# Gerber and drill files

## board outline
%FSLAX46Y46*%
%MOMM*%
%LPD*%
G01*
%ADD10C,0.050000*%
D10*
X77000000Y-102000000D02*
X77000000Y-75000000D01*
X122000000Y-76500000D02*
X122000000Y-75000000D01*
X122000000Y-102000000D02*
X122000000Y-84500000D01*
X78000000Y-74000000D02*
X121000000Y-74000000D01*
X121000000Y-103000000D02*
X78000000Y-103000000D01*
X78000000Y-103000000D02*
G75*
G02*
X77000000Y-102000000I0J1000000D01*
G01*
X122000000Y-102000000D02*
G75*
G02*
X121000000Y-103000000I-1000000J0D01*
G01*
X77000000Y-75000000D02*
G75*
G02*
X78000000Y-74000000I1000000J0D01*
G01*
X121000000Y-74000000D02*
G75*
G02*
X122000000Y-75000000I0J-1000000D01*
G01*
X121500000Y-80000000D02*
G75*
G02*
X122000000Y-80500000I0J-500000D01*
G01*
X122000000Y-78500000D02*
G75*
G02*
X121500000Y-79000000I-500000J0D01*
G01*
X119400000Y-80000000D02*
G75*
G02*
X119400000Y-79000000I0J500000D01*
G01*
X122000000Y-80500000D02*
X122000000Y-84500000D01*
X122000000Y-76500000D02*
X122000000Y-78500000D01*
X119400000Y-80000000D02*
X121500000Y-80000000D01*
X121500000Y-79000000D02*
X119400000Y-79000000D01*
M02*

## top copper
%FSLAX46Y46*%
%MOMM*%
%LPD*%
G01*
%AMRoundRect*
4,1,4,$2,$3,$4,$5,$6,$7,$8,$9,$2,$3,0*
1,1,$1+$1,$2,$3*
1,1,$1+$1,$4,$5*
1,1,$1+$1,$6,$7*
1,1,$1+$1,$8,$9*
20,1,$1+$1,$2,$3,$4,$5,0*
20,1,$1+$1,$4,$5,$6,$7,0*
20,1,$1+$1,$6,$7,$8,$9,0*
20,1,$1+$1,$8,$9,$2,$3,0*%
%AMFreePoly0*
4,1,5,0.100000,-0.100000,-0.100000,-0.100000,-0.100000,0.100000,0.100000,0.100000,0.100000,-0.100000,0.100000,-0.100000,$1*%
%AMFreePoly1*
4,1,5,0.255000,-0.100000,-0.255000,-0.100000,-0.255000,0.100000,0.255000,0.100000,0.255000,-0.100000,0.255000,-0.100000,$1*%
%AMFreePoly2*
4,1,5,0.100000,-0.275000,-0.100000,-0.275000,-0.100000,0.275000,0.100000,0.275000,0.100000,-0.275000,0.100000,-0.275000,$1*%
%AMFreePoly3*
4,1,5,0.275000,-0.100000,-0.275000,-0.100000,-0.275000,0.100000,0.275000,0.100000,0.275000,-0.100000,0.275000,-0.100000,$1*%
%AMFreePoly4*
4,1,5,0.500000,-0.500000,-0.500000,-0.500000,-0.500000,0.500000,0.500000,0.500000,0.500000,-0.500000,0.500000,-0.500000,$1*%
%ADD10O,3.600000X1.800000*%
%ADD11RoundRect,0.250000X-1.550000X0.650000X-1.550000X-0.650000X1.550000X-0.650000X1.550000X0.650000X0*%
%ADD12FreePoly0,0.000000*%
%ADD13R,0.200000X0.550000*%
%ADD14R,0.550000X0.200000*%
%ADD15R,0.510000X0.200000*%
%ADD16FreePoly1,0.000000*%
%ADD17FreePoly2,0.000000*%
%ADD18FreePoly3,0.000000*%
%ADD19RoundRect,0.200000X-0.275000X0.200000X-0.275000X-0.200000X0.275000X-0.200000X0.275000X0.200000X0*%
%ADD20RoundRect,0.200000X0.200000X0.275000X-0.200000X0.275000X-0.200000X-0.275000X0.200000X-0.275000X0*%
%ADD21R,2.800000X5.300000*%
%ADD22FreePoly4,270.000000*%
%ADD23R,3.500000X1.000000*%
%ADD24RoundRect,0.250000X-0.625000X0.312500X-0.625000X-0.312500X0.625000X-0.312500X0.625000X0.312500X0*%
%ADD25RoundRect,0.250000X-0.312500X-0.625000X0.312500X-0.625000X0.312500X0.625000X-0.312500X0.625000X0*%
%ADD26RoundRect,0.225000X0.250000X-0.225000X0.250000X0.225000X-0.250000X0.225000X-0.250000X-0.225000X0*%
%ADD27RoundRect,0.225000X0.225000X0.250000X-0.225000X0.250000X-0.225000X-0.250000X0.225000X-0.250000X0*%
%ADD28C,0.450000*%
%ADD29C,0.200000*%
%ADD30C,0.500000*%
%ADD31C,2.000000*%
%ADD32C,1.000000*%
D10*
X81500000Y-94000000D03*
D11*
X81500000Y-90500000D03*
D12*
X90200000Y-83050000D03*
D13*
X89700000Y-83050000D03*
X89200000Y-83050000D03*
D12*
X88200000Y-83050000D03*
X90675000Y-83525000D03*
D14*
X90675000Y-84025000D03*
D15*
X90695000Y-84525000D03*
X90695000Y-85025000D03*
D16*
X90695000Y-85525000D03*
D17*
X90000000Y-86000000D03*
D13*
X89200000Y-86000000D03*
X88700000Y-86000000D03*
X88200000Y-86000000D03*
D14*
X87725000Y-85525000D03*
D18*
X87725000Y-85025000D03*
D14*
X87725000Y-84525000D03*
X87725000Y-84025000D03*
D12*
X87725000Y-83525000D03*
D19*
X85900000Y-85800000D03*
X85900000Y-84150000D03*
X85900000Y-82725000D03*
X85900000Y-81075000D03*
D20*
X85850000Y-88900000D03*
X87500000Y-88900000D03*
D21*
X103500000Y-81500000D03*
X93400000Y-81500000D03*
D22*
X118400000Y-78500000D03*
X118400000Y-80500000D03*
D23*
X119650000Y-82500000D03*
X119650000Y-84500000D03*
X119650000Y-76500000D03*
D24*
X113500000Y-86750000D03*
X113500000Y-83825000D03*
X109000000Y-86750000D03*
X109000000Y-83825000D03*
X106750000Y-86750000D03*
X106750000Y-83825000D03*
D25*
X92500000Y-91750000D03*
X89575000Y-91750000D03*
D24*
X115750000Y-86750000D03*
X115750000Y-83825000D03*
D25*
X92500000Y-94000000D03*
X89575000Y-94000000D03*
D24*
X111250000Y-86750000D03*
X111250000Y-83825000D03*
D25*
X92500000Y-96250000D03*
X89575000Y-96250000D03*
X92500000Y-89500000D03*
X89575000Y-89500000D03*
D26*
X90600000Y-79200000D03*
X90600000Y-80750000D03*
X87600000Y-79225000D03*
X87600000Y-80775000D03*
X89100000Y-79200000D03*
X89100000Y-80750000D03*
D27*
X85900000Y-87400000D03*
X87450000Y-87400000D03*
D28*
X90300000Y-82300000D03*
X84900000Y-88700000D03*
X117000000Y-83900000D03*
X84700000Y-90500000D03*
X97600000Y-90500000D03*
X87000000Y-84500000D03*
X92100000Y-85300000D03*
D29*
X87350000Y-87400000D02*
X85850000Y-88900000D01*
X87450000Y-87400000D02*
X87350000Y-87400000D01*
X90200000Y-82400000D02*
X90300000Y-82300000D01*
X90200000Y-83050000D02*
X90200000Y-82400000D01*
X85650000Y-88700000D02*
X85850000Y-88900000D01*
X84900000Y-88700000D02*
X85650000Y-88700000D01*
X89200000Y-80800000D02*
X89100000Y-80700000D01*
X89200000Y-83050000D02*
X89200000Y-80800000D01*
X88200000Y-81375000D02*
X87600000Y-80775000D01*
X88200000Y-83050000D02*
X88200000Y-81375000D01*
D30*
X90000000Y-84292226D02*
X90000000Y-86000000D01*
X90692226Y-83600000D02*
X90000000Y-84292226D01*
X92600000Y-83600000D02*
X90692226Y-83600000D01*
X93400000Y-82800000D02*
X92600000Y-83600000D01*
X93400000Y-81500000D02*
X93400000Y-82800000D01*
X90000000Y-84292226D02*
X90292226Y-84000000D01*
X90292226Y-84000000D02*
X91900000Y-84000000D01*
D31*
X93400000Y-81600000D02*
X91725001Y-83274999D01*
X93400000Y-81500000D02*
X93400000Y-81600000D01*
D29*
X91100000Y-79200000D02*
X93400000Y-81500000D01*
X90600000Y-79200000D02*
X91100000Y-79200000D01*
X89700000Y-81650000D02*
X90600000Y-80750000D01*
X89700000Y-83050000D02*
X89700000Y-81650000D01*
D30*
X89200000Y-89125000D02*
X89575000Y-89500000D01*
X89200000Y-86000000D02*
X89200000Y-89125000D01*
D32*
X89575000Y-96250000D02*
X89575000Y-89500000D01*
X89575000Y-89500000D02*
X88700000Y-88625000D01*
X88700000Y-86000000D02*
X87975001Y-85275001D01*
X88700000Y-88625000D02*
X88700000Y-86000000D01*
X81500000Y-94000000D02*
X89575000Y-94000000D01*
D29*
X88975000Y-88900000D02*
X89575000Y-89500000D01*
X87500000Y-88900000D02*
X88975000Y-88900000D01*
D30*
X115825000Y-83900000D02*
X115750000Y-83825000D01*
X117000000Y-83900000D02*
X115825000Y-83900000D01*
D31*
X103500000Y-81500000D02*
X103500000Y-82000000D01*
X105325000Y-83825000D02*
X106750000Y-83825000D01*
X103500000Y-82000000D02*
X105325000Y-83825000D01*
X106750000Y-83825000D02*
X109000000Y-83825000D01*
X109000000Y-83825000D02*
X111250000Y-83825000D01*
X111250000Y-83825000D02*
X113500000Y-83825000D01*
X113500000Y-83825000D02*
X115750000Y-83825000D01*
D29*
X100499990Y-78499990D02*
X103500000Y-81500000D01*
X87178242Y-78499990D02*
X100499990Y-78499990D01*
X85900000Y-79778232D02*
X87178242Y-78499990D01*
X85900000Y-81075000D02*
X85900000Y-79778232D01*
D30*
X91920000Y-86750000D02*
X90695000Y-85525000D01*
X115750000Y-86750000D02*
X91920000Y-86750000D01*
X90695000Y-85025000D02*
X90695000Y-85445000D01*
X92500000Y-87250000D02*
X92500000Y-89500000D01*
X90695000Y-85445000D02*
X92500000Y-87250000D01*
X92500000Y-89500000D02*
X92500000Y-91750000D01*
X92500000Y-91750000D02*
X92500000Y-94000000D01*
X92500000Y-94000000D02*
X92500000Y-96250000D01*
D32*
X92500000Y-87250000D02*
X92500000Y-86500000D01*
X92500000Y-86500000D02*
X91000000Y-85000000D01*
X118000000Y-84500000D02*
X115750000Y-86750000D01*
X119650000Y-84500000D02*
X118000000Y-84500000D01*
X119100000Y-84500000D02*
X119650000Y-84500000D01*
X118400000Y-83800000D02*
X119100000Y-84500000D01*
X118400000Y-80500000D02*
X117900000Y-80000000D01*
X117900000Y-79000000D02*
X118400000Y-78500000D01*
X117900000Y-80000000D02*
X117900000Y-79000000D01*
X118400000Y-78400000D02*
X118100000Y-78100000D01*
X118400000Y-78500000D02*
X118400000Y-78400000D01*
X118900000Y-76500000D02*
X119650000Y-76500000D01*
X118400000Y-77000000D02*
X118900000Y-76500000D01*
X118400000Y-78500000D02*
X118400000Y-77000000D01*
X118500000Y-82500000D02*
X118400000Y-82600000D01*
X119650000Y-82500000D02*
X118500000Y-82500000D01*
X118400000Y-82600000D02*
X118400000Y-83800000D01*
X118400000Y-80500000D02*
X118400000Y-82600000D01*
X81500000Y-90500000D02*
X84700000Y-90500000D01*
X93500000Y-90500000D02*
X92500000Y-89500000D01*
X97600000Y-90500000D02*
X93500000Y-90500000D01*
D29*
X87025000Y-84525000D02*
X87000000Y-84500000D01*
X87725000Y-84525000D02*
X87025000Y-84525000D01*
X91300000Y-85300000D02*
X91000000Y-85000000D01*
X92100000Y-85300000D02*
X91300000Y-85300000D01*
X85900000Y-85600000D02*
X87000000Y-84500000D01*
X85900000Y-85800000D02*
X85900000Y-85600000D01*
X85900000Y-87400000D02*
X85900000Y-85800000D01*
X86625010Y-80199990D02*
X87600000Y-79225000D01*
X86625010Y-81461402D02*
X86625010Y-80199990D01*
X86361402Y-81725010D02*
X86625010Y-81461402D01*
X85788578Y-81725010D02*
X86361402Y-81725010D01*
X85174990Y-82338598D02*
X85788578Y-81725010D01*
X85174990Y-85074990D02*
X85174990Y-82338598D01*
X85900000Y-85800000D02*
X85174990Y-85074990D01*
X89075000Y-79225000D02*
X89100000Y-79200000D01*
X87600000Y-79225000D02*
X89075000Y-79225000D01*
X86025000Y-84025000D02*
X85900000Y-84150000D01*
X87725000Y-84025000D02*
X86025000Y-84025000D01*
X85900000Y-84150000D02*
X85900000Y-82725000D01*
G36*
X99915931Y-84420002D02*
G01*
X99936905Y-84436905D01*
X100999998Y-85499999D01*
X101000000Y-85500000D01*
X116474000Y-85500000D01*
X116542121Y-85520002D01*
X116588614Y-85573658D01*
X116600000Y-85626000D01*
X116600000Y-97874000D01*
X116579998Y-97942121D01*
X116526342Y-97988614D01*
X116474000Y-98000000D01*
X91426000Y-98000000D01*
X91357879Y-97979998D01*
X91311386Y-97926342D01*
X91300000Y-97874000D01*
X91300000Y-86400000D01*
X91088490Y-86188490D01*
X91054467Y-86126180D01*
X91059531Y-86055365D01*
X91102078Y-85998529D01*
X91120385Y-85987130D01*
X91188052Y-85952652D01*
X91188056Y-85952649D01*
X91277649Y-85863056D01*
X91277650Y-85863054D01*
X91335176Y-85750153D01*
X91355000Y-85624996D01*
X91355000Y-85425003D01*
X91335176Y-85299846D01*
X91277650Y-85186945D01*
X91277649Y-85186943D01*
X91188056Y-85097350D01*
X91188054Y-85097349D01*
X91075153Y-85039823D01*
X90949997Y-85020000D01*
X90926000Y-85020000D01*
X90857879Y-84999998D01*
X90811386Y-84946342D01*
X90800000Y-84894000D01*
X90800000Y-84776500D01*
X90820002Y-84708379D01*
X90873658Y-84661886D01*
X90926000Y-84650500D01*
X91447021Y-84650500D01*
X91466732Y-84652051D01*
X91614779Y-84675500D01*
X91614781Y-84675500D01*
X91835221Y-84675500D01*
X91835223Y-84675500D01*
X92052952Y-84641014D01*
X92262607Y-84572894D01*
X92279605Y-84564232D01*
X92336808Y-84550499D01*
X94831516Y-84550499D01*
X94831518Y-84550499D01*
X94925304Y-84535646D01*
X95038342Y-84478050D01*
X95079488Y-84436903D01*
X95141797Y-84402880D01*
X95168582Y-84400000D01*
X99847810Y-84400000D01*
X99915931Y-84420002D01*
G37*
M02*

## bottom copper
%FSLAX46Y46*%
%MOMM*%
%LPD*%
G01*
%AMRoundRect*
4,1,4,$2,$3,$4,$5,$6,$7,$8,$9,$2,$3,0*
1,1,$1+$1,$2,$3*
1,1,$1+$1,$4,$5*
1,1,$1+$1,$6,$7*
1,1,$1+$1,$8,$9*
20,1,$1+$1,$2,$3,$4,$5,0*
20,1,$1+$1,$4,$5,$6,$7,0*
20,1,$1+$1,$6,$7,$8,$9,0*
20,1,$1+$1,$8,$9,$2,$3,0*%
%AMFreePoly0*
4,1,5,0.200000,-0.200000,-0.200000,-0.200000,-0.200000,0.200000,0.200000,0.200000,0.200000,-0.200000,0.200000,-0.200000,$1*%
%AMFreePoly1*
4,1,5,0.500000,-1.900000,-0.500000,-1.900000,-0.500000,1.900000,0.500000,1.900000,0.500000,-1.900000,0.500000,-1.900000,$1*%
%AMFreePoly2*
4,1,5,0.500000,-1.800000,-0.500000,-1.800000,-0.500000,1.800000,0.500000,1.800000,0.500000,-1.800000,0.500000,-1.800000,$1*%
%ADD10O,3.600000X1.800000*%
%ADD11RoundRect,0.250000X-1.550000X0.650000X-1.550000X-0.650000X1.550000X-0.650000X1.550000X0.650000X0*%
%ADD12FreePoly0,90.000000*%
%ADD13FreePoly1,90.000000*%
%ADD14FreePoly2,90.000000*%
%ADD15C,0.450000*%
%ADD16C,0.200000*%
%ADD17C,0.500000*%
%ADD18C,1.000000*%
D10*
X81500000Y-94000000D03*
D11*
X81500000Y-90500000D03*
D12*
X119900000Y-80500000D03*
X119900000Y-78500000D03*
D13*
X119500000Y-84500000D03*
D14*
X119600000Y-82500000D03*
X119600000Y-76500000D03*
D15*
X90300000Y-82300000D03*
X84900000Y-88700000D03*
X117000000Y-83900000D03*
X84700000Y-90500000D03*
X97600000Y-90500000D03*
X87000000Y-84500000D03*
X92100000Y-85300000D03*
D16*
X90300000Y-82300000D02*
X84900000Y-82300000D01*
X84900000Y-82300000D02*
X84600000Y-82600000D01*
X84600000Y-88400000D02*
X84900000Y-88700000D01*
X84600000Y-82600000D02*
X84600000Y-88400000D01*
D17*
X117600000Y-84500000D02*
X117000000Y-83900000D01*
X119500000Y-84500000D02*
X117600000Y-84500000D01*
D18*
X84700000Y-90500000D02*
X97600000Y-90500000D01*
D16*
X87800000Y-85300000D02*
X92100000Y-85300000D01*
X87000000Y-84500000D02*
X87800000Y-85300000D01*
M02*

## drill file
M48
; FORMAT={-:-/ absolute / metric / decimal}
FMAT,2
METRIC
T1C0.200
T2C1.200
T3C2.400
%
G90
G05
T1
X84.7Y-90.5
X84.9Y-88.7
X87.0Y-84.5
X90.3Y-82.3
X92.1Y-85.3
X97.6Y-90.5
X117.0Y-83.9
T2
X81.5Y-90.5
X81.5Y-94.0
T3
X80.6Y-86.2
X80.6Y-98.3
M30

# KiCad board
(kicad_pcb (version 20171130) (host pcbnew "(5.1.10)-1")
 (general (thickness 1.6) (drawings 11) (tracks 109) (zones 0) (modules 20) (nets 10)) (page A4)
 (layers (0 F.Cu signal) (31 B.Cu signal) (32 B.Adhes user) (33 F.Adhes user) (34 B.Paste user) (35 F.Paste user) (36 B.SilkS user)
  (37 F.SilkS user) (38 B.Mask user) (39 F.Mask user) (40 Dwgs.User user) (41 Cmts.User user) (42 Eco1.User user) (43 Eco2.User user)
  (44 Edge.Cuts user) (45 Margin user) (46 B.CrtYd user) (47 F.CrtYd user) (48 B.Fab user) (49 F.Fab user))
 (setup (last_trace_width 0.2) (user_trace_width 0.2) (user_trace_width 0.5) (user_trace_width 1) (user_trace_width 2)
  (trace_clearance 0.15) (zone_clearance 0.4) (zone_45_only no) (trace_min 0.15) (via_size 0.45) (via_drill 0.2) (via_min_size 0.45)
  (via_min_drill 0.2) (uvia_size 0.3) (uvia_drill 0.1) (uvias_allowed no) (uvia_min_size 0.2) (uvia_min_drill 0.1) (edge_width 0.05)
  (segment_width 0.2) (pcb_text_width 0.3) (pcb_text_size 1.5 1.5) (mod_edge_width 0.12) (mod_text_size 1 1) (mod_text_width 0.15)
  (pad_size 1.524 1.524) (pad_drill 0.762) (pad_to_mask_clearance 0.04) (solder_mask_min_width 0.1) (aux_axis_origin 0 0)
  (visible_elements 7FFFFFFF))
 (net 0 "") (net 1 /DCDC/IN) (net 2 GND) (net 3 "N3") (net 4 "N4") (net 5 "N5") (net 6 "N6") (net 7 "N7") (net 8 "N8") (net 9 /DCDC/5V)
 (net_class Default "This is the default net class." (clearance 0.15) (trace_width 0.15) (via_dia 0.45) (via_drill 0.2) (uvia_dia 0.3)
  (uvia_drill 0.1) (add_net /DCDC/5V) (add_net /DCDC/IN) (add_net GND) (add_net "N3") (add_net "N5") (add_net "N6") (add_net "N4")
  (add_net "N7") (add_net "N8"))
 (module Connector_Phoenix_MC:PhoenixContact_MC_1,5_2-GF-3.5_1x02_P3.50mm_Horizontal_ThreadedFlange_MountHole (layer F.Cu)
  (at 81.5 90.5 270)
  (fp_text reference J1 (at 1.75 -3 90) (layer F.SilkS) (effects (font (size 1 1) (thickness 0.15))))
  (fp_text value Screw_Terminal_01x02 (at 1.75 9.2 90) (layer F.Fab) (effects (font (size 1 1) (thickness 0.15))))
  (pad "" np_thru_hole circle (at 7.8 0.9 270) (size 2.4 2.4) (drill 2.4) (layers *.Cu *.Mask))
  (pad "" np_thru_hole circle (at -4.3 0.9 270) (size 2.4 2.4) (drill 2.4) (layers *.Cu *.Mask))
  (pad 2 thru_hole oval (at 3.5 0 270) (size 1.8 3.6) (drill 1.2) (layers *.Cu *.Mask) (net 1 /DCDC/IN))
  (pad 1 thru_hole roundrect (at 0 0 270) (size 1.8 3.6) (drill 1.2) (layers *.Cu *.Mask) (roundrect_rratio 0.138889) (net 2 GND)))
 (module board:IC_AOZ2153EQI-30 (layer F.Cu) (at 89.2 84.525)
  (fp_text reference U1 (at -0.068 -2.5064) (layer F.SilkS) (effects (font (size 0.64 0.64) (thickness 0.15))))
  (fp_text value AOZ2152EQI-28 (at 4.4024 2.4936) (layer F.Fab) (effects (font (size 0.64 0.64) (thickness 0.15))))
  (pad 15 smd custom (at 1 -1.475) (size 0.2 0.2) (layers F.Cu) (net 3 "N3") (zone_connect 0) (options (clearance outline) (anchor rect))
   (primitives))
  (pad 16 smd rect (at 0.5 -1.475) (size 0.2 0.55) (layers F.Cu F.Paste F.Mask) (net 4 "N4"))
  (pad 17 smd rect (at 0 -1.475) (size 0.2 0.55) (layers F.Cu F.Paste F.Mask) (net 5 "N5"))
  (pad 18 smd custom (at -1 -1.475) (size 0.2 0.2) (layers F.Cu) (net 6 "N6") (zone_connect 0) (options (clearance outline) (anchor rect))
   (primitives))
  (pad 14 smd custom (at 1.475 -1) (size 0.2 0.2) (layers F.Cu) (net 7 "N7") (zone_connect 0) (options (clearance outline) (anchor rect))
   (primitives))
  (pad 13 smd rect (at 1.475 -0.5) (size 0.55 0.2) (layers F.Cu F.Paste) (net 7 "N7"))
  (pad 12 smd rect (at 1.495 0) (size 0.51 0.2) (layers F.Cu F.Paste) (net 2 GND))
  (pad 11 smd rect (at 1.495 0.5) (size 0.51 0.2) (layers F.Cu F.Paste) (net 2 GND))
  (pad 10 smd custom (at 1.495 1) (size 0.51 0.2) (layers F.Cu F.Paste) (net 2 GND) (zone_connect 0)
   (options (clearance outline) (anchor rect)) (primitives))
  (pad 9 smd custom (at 0.8 1.475) (size 0.2 0.55) (layers F.Cu F.Paste) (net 7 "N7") (zone_connect 0)
   (options (clearance outline) (anchor rect)) (primitives))
  (pad 8 smd rect (at 0 1.475) (size 0.2 0.55) (layers F.Cu F.Paste) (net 1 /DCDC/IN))
  (pad 7 smd rect (at -0.5 1.475) (size 0.2 0.55) (layers F.Cu F.Paste) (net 1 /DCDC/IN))
  (pad 6 smd rect (at -1 1.475) (size 0.2 0.55) (layers F.Cu F.Paste) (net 1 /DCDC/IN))
  (pad 5 smd rect (at -1.475 1) (size 0.55 0.2) (layers F.Cu F.Paste) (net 1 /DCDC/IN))
  (pad 4 smd custom (at -1.475 0.5) (size 0.55 0.2) (layers F.Cu F.Paste) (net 1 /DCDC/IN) (zone_connect 0)
   (options (clearance outline) (anchor rect)) (primitives))
  (pad 3 smd rect (at -1.475 0) (size 0.55 0.2) (layers F.Cu F.Paste F.Mask) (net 2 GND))
  (pad 2 smd rect (at -1.475 -0.5) (size 0.55 0.2) (layers F.Cu F.Paste F.Mask) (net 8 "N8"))
  (pad 1 smd custom (at -1.475 -1) (size 0.2 0.2) (layers F.Cu) (zone_connect 0) (options (clearance outline) (anchor rect)) (primitives)))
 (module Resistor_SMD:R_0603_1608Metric (layer F.Cu) (at 85.9 84.975 270)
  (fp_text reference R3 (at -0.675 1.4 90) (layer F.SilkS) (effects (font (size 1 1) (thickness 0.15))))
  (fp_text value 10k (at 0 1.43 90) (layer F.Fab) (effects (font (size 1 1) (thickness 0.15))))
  (pad 2 smd roundrect (at 0.825 0 270) (size 0.8 0.95) (layers F.Cu F.Paste F.Mask) (roundrect_rratio 0.25) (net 2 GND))
  (pad 1 smd roundrect (at -0.825 0 270) (size 0.8 0.95) (layers F.Cu F.Paste F.Mask) (roundrect_rratio 0.25) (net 8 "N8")))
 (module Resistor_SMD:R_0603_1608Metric (layer F.Cu) (at 85.9 81.9 270)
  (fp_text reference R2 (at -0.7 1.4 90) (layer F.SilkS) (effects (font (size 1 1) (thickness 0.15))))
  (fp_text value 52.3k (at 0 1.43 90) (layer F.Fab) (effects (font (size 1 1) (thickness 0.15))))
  (pad 2 smd roundrect (at 0.825 0 270) (size 0.8 0.95) (layers F.Cu F.Paste F.Mask) (roundrect_rratio 0.25) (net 8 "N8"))
  (pad 1 smd roundrect (at -0.825 0 270) (size 0.8 0.95) (layers F.Cu F.Paste F.Mask) (roundrect_rratio 0.25) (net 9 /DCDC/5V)))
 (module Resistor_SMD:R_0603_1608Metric (layer F.Cu) (at 86.675 88.9 180)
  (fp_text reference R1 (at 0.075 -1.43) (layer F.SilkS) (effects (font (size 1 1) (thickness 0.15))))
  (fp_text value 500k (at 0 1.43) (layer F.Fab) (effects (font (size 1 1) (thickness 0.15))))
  (pad 2 smd roundrect (at 0.825 0 180) (size 0.8 0.95) (layers F.Cu F.Paste F.Mask) (roundrect_rratio 0.25) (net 3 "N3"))
  (pad 1 smd roundrect (at -0.825 0 180) (size 0.8 0.95) (layers F.Cu F.Paste F.Mask) (roundrect_rratio 0.25) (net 1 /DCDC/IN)))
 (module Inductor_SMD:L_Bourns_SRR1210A (layer F.Cu) (at 98.45 81.5 180)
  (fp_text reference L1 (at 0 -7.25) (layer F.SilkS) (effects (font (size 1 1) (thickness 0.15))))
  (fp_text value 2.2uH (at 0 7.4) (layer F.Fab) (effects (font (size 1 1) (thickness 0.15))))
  (pad 1 smd rect (at -5.05 0 180) (size 2.8 5.3) (layers F.Cu F.Paste F.Mask) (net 9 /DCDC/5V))
  (pad 2 smd rect (at 5.05 0 180) (size 2.8 5.3) (layers F.Cu F.Paste F.Mask) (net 7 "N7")))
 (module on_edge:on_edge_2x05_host (layer F.Cu) (at 122 80.5 270)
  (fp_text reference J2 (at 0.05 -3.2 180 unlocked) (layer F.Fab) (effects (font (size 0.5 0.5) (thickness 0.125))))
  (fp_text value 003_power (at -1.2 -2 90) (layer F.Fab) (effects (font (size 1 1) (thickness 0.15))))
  (fp_arc (start 0 0.5) (end 0 0) (angle -90) (layer Edge.Cuts) (width 0.05))
  (fp_arc (start -2 0.5) (end -1.5 0.5) (angle -90) (layer Edge.Cuts) (width 0.05))
  (fp_arc (start -1 2.6) (end -1.5 2.6) (angle -180) (layer Edge.Cuts) (width 0.05))
  (fp_line (start 0 0) (end 4 0) (layer Edge.Cuts) (width 0.05))
  (fp_line (start -4 0) (end -2 0) (layer Edge.Cuts) (width 0.05))
  (fp_line (start -0.5 2.6) (end -0.5 0.5) (layer Edge.Cuts) (width 0.05))
  (fp_line (start -1.5 0.5) (end -1.5 2.6) (layer Edge.Cuts) (width 0.05))
  (pad 2 smd custom (at -2 3.6 270) (size 1 1) (layers F.Cu F.Mask) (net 2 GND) (zone_connect 0) (options (clearance outline) (anchor rect))
   (primitives))
  (pad 3 smd custom (at 0 3.6 270) (size 1 1) (layers F.Cu F.Mask) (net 2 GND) (zone_connect 0) (options (clearance outline) (anchor rect))
   (primitives))
  (pad 8 smd custom (at 0 2.1 90) (size 0.4 0.4) (layers B.Cu B.Mask) (zone_connect 0) (options (clearance outline) (anchor rect))
   (primitives))
  (pad 7 smd custom (at -2 2.1 90) (size 0.4 0.4) (layers B.Cu B.Mask) (zone_connect 0) (options (clearance outline) (anchor rect))
   (primitives))
  (pad 4 smd rect (at 2 2.35 270) (size 1 3.5) (layers F.Cu F.Mask) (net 2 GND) (zone_connect 0))
  (pad 10 smd custom (at 4 2.5 90) (size 1 3.8) (layers B.Cu B.Mask) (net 9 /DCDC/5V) (zone_connect 0)
   (options (clearance outline) (anchor rect)) (primitives))
  (pad 9 smd custom (at 2 2.4 90) (size 1 3.6) (layers B.Cu B.Mask) (zone_connect 0) (options (clearance outline) (anchor rect))
   (primitives))
  (pad 6 smd custom (at -4 2.4 90) (size 1 3.6) (layers B.Cu B.Mask) (zone_connect 0) (options (clearance outline) (anchor rect))
   (primitives))
  (pad 5 smd rect (at 4 2.35 270) (size 1 3.5) (layers F.Cu F.Mask) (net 2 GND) (zone_connect 0))
  (pad 1 smd rect (at -4 2.35 270) (size 1 3.5) (layers F.Cu F.Mask) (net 2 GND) (zone_connect 0)))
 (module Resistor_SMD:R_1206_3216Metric (layer F.Cu) (at 113.5 85.2875 270)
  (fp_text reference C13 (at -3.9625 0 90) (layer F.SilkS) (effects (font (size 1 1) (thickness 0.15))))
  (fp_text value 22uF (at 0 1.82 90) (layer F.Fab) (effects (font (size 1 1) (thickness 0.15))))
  (pad 2 smd roundrect (at 1.4625 0 270) (size 1.125 1.75) (layers F.Cu F.Paste F.Mask) (roundrect_rratio 0.222222) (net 2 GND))
  (pad 1 smd roundrect (at -1.4625 0 270) (size 1.125 1.75) (layers F.Cu F.Paste F.Mask) (roundrect_rratio 0.222222) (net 9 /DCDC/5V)))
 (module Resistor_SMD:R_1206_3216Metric (layer F.Cu) (at 109 85.2875 270)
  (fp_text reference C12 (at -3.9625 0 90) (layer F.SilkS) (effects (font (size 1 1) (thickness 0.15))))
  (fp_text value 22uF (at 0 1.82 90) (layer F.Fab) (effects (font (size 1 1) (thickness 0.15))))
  (pad 2 smd roundrect (at 1.4625 0 270) (size 1.125 1.75) (layers F.Cu F.Paste F.Mask) (roundrect_rratio 0.222222) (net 2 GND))
  (pad 1 smd roundrect (at -1.4625 0 270) (size 1.125 1.75) (layers F.Cu F.Paste F.Mask) (roundrect_rratio 0.222222) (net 9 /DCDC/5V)))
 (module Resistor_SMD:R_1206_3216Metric (layer F.Cu) (at 106.75 85.2875 270)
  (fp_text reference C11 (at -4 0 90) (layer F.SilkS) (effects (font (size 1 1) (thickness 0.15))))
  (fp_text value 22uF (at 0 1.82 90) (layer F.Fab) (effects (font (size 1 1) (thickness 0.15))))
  (pad 2 smd roundrect (at 1.4625 0 270) (size 1.125 1.75) (layers F.Cu F.Paste F.Mask) (roundrect_rratio 0.222222) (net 2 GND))
  (pad 1 smd roundrect (at -1.4625 0 270) (size 1.125 1.75) (layers F.Cu F.Paste F.Mask) (roundrect_rratio 0.222222) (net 9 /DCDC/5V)))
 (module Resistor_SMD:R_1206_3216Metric (layer F.Cu) (at 91.0375 91.75)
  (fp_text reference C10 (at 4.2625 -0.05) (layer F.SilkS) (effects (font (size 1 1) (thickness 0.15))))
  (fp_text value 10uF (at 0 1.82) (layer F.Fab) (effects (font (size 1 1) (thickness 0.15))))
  (pad 2 smd roundrect (at 1.4625 0) (size 1.125 1.75) (layers F.Cu F.Paste F.Mask) (roundrect_rratio 0.222222) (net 2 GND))
  (pad 1 smd roundrect (at -1.4625 0) (size 1.125 1.75) (layers F.Cu F.Paste F.Mask) (roundrect_rratio 0.222222) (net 1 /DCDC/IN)))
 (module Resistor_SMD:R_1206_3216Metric (layer F.Cu) (at 115.75 85.2875 270)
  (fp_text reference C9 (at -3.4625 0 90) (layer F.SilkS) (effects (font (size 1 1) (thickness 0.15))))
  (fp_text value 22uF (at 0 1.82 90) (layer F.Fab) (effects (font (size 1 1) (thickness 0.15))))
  (pad 2 smd roundrect (at 1.4625 0 270) (size 1.125 1.75) (layers F.Cu F.Paste F.Mask) (roundrect_rratio 0.222222) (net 2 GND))
  (pad 1 smd roundrect (at -1.4625 0 270) (size 1.125 1.75) (layers F.Cu F.Paste F.Mask) (roundrect_rratio 0.222222) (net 9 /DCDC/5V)))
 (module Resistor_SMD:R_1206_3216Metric (layer F.Cu) (at 91.0375 94)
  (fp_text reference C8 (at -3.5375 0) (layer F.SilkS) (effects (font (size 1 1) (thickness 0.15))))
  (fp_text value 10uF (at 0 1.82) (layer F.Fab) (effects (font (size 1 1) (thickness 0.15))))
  (pad 2 smd roundrect (at 1.4625 0) (size 1.125 1.75) (layers F.Cu F.Paste F.Mask) (roundrect_rratio 0.222222) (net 2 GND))
  (pad 1 smd roundrect (at -1.4625 0) (size 1.125 1.75) (layers F.Cu F.Paste F.Mask) (roundrect_rratio 0.222222) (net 1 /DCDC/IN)))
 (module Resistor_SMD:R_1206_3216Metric (layer F.Cu) (at 111.25 85.2875 270)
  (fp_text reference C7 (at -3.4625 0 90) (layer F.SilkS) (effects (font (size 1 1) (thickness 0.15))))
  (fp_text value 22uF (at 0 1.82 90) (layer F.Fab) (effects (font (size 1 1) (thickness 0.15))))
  (pad 2 smd roundrect (at 1.4625 0 270) (size 1.125 1.75) (layers F.Cu F.Paste F.Mask) (roundrect_rratio 0.222222) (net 2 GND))
  (pad 1 smd roundrect (at -1.4625 0 270) (size 1.125 1.75) (layers F.Cu F.Paste F.Mask) (roundrect_rratio 0.222222) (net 9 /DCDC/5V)))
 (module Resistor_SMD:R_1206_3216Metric (layer F.Cu) (at 91.0375 96.25)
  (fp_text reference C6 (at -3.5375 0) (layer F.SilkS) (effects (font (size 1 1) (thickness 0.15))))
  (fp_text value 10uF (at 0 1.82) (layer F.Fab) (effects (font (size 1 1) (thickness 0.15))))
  (pad 2 smd roundrect (at 1.4625 0) (size 1.125 1.75) (layers F.Cu F.Paste F.Mask) (roundrect_rratio 0.222222) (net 2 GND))
  (pad 1 smd roundrect (at -1.4625 0) (size 1.125 1.75) (layers F.Cu F.Paste F.Mask) (roundrect_rratio 0.222222) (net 1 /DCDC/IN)))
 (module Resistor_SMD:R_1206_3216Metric (layer F.Cu) (at 91.0375 89.5)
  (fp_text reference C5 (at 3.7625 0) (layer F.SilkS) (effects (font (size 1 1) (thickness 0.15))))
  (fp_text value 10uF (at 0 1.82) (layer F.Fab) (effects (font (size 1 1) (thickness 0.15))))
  (pad 2 smd roundrect (at 1.4625 0) (size 1.125 1.75) (layers F.Cu F.Paste F.Mask) (roundrect_rratio 0.222222) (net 2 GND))
  (pad 1 smd roundrect (at -1.4625 0) (size 1.125 1.75) (layers F.Cu F.Paste F.Mask) (roundrect_rratio 0.222222) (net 1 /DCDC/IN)))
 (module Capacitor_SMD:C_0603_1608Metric (layer F.Cu) (at 90.6 79.975 90)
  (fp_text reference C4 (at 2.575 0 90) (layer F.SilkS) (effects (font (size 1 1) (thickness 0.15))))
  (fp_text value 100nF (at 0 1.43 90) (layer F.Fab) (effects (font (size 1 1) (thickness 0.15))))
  (pad 2 smd roundrect (at 0.775 0 90) (size 0.9 0.95) (layers F.Cu F.Paste F.Mask) (roundrect_rratio 0.25) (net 7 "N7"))
  (pad 1 smd roundrect (at -0.775 0 90) (size 0.9 0.95) (layers F.Cu F.Paste F.Mask) (roundrect_rratio 0.25) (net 4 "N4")))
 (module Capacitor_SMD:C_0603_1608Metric (layer F.Cu) (at 87.6 80 90)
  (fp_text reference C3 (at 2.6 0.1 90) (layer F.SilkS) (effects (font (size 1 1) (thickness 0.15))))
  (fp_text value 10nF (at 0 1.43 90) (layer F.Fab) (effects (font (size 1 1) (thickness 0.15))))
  (pad 2 smd roundrect (at 0.775 0 90) (size 0.9 0.95) (layers F.Cu F.Paste F.Mask) (roundrect_rratio 0.25) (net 2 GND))
  (pad 1 smd roundrect (at -0.775 0 90) (size 0.9 0.95) (layers F.Cu F.Paste F.Mask) (roundrect_rratio 0.25) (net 6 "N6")))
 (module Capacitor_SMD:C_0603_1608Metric (layer F.Cu) (at 89.1 79.975 90)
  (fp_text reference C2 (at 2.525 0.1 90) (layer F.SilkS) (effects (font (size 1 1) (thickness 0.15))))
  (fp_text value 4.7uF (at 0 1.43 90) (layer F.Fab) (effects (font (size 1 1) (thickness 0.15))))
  (pad 2 smd roundrect (at 0.775 0 90) (size 0.9 0.95) (layers F.Cu F.Paste F.Mask) (roundrect_rratio 0.25) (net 2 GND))
  (pad 1 smd roundrect (at -0.775 0 90) (size 0.9 0.95) (layers F.Cu F.Paste F.Mask) (roundrect_rratio 0.25) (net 5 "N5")))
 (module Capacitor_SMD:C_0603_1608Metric (layer F.Cu) (at 86.675 87.4 180)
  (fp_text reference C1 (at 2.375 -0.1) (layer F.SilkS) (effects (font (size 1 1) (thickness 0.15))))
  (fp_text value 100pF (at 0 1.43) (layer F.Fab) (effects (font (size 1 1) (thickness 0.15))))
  (pad 2 smd roundrect (at 0.775 0 180) (size 0.9 0.95) (layers F.Cu F.Paste F.Mask) (roundrect_rratio 0.25) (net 2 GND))
  (pad 1 smd roundrect (at -0.775 0 180) (size 0.9 0.95) (layers F.Cu F.Paste F.Mask) (roundrect_rratio 0.25) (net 3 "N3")))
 (gr_line (start 77 102) (end 77 75) (layer Edge.Cuts) (width 0.05))
 (gr_line (start 122 76.5) (end 122 75) (layer Edge.Cuts) (width 0.05))
 (gr_line (start 122 102) (end 122 84.5) (layer Edge.Cuts) (width 0.05))
 (gr_line (start 78 74) (end 121 74) (layer Edge.Cuts) (width 0.05))
 (gr_line (start 121 103) (end 78 103) (layer Edge.Cuts) (width 0.05))
 (gr_arc (start 78 102) (end 77 102) (angle -90) (layer Edge.Cuts) (width 0.05))
 (gr_arc (start 121 102) (end 121 103) (angle -90) (layer Edge.Cuts) (width 0.05))
 (gr_arc (start 78 75) (end 78 74) (angle -90) (layer Edge.Cuts) (width 0.05))
 (gr_arc (start 121 75) (end 122 75) (angle -90) (layer Edge.Cuts) (width 0.05))
 (segment (start 87.35 87.4) (end 85.85 88.9) (width 0.2) (layer F.Cu) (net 3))
 (segment (start 87.45 87.4) (end 87.35 87.4) (width 0.2) (layer F.Cu) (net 3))
 (via (at 90.3 82.3) (size 0.45) (drill 0.2) (layers F.Cu B.Cu) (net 3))
 (segment (start 90.2 82.4) (end 90.3 82.3) (width 0.2) (layer F.Cu) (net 3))
 (segment (start 90.2 83.05) (end 90.2 82.4) (width 0.2) (layer F.Cu) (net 3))
 (segment (start 90.3 82.3) (end 84.9 82.3) (width 0.2) (layer B.Cu) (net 3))
 (segment (start 84.9 82.3) (end 84.6 82.6) (width 0.2) (layer B.Cu) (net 3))
 (via (at 84.9 88.7) (size 0.45) (drill 0.2) (layers F.Cu B.Cu) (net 3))
 (segment (start 84.6 88.4) (end 84.9 88.7) (width 0.2) (layer B.Cu) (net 3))
 (segment (start 84.6 82.6) (end 84.6 88.4) (width 0.2) (layer B.Cu) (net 3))
 (segment (start 85.65 88.7) (end 85.85 88.9) (width 0.2) (layer F.Cu) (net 3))
 (segment (start 84.9 88.7) (end 85.65 88.7) (width 0.2) (layer F.Cu) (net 3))
 (segment (start 89.2 80.8) (end 89.1 80.7) (width 0.2) (layer F.Cu) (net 5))
 (segment (start 89.2 83.05) (end 89.2 80.8) (width 0.2) (layer F.Cu) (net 5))
 (segment (start 88.2 81.375) (end 87.6 80.775) (width 0.2) (layer F.Cu) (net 6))
 (segment (start 88.2 83.05) (end 88.2 81.375) (width 0.2) (layer F.Cu) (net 6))
 (segment (start 90 84.292226) (end 90 86) (width 0.5) (layer F.Cu) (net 7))
 (segment (start 90.692226 83.6) (end 90 84.292226) (width 0.5) (layer F.Cu) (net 7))
 (segment (start 92.6 83.6) (end 90.692226 83.6) (width 0.5) (layer F.Cu) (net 7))
 (segment (start 93.4 82.8) (end 92.6 83.6) (width 0.5) (layer F.Cu) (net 7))
 (segment (start 93.4 81.5) (end 93.4 82.8) (width 0.5) (layer F.Cu) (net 7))
 (segment (start 90 84.292226) (end 90.292226 84) (width 0.5) (layer F.Cu) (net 7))
 (segment (start 90.292226 84) (end 91.9 84) (width 0.5) (layer F.Cu) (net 7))
 (segment (start 93.4 81.6) (end 91.725001 83.274999) (width 2) (layer F.Cu) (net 7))
 (segment (start 93.4 81.5) (end 93.4 81.6) (width 2) (layer F.Cu) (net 7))
 (segment (start 91.1 79.2) (end 93.4 81.5) (width 0.2) (layer F.Cu) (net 7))
 (segment (start 90.6 79.2) (end 91.1 79.2) (width 0.2) (layer F.Cu) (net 7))
 (segment (start 89.7 81.65) (end 90.6 80.75) (width 0.2) (layer F.Cu) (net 4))
 (segment (start 89.7 83.05) (end 89.7 81.65) (width 0.2) (layer F.Cu) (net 4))
 (segment (start 89.2 89.125) (end 89.575 89.5) (width 0.5) (layer F.Cu) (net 1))
 (segment (start 89.2 86) (end 89.2 89.125) (width 0.5) (layer F.Cu) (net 1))
 (segment (start 89.575 96.25) (end 89.575 89.5) (width 1) (layer F.Cu) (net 1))
 (segment (start 89.575 89.5) (end 88.7 88.625) (width 1) (layer F.Cu) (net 1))
 (segment (start 88.7 86) (end 87.975001 85.275001) (width 1) (layer F.Cu) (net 1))
 (segment (start 88.7 88.625) (end 88.7 86) (width 1) (layer F.Cu) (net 1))
 (segment (start 81.5 94) (end 89.575 94) (width 1) (layer F.Cu) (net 1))
 (segment (start 88.975 88.9) (end 89.575 89.5) (width 0.2) (layer F.Cu) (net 1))
 (segment (start 87.5 88.9) (end 88.975 88.9) (width 0.2) (layer F.Cu) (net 1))
 (via (at 117 83.9) (size 0.45) (drill 0.2) (layers F.Cu B.Cu) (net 9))
 (segment (start 117.6 84.5) (end 117 83.9) (width 0.5) (layer B.Cu) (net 9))
 (segment (start 119.5 84.5) (end 117.6 84.5) (width 0.5) (layer B.Cu) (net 9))
 (segment (start 115.825 83.9) (end 115.75 83.825) (width 0.5) (layer F.Cu) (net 9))
 (segment (start 117 83.9) (end 115.825 83.9) (width 0.5) (layer F.Cu) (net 9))
 (segment (start 103.5 81.5) (end 103.5 82) (width 2) (layer F.Cu) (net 9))
 (segment (start 105.325 83.825) (end 106.75 83.825) (width 2) (layer F.Cu) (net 9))
 (segment (start 103.5 82) (end 105.325 83.825) (width 2) (layer F.Cu) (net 9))
 (segment (start 106.75 83.825) (end 109 83.825) (width 2) (layer F.Cu) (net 9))
 (segment (start 109 83.825) (end 111.25 83.825) (width 2) (layer F.Cu) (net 9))
 (segment (start 111.25 83.825) (end 113.5 83.825) (width 2) (layer F.Cu) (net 9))
 (segment (start 113.5 83.825) (end 115.75 83.825) (width 2) (layer F.Cu) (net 9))
 (segment (start 100.49999 78.49999) (end 103.5 81.5) (width 0.2) (layer F.Cu) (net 9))
 (segment (start 87.178242 78.49999) (end 100.49999 78.49999) (width 0.2) (layer F.Cu) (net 9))
 (segment (start 85.9 79.778232) (end 87.178242 78.49999) (width 0.2) (layer F.Cu) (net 9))
 (segment (start 85.9 81.075) (end 85.9 79.778232) (width 0.2) (layer F.Cu) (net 9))
 (segment (start 91.92 86.75) (end 90.695 85.525) (width 0.5) (layer F.Cu) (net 2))
 (segment (start 115.75 86.75) (end 91.92 86.75) (width 0.5) (layer F.Cu) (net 2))
 (segment (start 90.695 85.025) (end 90.695 85.445) (width 0.5) (layer F.Cu) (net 2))
 (segment (start 92.5 87.25) (end 92.5 89.5) (width 0.5) (layer F.Cu) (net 2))
 (segment (start 90.695 85.445) (end 92.5 87.25) (width 0.5) (layer F.Cu) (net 2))
 (segment (start 92.5 89.5) (end 92.5 91.75) (width 0.5) (layer F.Cu) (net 2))
 (segment (start 92.5 91.75) (end 92.5 94) (width 0.5) (layer F.Cu) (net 2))
 (segment (start 92.5 94) (end 92.5 96.25) (width 0.5) (layer F.Cu) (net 2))
 (segment (start 92.5 87.25) (end 92.5 86.5) (width 1) (layer F.Cu) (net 2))
 (segment (start 92.5 86.5) (end 91 85) (width 1) (layer F.Cu) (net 2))
 (segment (start 118 84.5) (end 115.75 86.75) (width 1) (layer F.Cu) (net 2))
 (segment (start 119.65 84.5) (end 118 84.5) (width 1) (layer F.Cu) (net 2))
 (segment (start 119.1 84.5) (end 119.65 84.5) (width 1) (layer F.Cu) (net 2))
 (segment (start 118.4 83.8) (end 119.1 84.5) (width 1) (layer F.Cu) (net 2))
 (segment (start 118.4 80.5) (end 117.9 80) (width 1) (layer F.Cu) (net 2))
 (segment (start 117.9 79) (end 118.4 78.5) (width 1) (layer F.Cu) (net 2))
 (segment (start 117.9 80) (end 117.9 79) (width 1) (layer F.Cu) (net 2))
 (segment (start 118.4 78.4) (end 118.1 78.1) (width 1) (layer F.Cu) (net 2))
 (segment (start 118.4 78.5) (end 118.4 78.4) (width 1) (layer F.Cu) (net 2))
 (segment (start 118.9 76.5) (end 119.65 76.5) (width 1) (layer F.Cu) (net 2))
 (segment (start 118.4 77) (end 118.9 76.5) (width 1) (layer F.Cu) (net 2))
 (segment (start 118.4 78.5) (end 118.4 77) (width 1) (layer F.Cu) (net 2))
 (segment (start 118.5 82.5) (end 118.4 82.6) (width 1) (layer F.Cu) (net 2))
 (segment (start 119.65 82.5) (end 118.5 82.5) (width 1) (layer F.Cu) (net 2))
 (segment (start 118.4 82.6) (end 118.4 83.8) (width 1) (layer F.Cu) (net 2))
 (segment (start 118.4 80.5) (end 118.4 82.6) (width 1) (layer F.Cu) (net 2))
 (via (at 84.7 90.5) (size 0.45) (drill 0.2) (layers F.Cu B.Cu) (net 2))
 (segment (start 81.5 90.5) (end 84.7 90.5) (width 1) (layer F.Cu) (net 2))
 (via (at 97.6 90.5) (size 0.45) (drill 0.2) (layers F.Cu B.Cu) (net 2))
 (segment (start 84.7 90.5) (end 97.6 90.5) (width 1) (layer B.Cu) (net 2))
 (segment (start 93.5 90.5) (end 92.5 89.5) (width 1) (layer F.Cu) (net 2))
 (segment (start 97.6 90.5) (end 93.5 90.5) (width 1) (layer F.Cu) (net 2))
 (via (at 87 84.5) (size 0.45) (drill 0.2) (layers F.Cu B.Cu) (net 2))
 (segment (start 87.025 84.525) (end 87 84.5) (width 0.2) (layer F.Cu) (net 2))
 (segment (start 87.725 84.525) (end 87.025 84.525) (width 0.2) (layer F.Cu) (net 2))
 (via (at 92.1 85.3) (size 0.45) (drill 0.2) (layers F.Cu B.Cu) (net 2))
 (segment (start 87.8 85.3) (end 92.1 85.3) (width 0.2) (layer B.Cu) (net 2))
 (segment (start 87 84.5) (end 87.8 85.3) (width 0.2) (layer B.Cu) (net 2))
 (segment (start 91.3 85.3) (end 91 85) (width 0.2) (layer F.Cu) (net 2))
 (segment (start 92.1 85.3) (end 91.3 85.3) (width 0.2) (layer F.Cu) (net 2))
 (segment (start 85.9 85.6) (end 87 84.5) (width 0.2) (layer F.Cu) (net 2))
 (segment (start 85.9 85.8) (end 85.9 85.6) (width 0.2) (layer F.Cu) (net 2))
 (segment (start 85.9 87.4) (end 85.9 85.8) (width 0.2) (layer F.Cu) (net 2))
 (segment (start 86.62501 80.19999) (end 87.6 79.225) (width 0.2) (layer F.Cu) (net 2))
 (segment (start 86.62501 81.461402) (end 86.62501 80.19999) (width 0.2) (layer F.Cu) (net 2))
 (segment (start 86.361402 81.72501) (end 86.62501 81.461402) (width 0.2) (layer F.Cu) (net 2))
 (segment (start 85.788578 81.72501) (end 86.361402 81.72501) (width 0.2) (layer F.Cu) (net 2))
 (segment (start 85.17499 82.338598) (end 85.788578 81.72501) (width 0.2) (layer F.Cu) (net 2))
 (segment (start 85.17499 85.07499) (end 85.17499 82.338598) (width 0.2) (layer F.Cu) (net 2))
 (segment (start 85.9 85.8) (end 85.17499 85.07499) (width 0.2) (layer F.Cu) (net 2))
 (segment (start 89.075 79.225) (end 89.1 79.2) (width 0.2) (layer F.Cu) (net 2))
 (segment (start 87.6 79.225) (end 89.075 79.225) (width 0.2) (layer F.Cu) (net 2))
 (segment (start 86.025 84.025) (end 85.9 84.15) (width 0.2) (layer F.Cu) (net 8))
 (segment (start 87.725 84.025) (end 86.025 84.025) (width 0.2) (layer F.Cu) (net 8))
 (segment (start 85.9 84.15) (end 85.9 82.725) (width 0.2) (layer F.Cu) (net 8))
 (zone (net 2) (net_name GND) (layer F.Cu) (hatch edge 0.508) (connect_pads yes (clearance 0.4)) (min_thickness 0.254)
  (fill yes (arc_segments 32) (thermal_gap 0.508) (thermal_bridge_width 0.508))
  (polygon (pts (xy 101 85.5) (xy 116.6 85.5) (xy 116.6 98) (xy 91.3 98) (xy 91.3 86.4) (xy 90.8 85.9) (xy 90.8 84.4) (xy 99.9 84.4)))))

